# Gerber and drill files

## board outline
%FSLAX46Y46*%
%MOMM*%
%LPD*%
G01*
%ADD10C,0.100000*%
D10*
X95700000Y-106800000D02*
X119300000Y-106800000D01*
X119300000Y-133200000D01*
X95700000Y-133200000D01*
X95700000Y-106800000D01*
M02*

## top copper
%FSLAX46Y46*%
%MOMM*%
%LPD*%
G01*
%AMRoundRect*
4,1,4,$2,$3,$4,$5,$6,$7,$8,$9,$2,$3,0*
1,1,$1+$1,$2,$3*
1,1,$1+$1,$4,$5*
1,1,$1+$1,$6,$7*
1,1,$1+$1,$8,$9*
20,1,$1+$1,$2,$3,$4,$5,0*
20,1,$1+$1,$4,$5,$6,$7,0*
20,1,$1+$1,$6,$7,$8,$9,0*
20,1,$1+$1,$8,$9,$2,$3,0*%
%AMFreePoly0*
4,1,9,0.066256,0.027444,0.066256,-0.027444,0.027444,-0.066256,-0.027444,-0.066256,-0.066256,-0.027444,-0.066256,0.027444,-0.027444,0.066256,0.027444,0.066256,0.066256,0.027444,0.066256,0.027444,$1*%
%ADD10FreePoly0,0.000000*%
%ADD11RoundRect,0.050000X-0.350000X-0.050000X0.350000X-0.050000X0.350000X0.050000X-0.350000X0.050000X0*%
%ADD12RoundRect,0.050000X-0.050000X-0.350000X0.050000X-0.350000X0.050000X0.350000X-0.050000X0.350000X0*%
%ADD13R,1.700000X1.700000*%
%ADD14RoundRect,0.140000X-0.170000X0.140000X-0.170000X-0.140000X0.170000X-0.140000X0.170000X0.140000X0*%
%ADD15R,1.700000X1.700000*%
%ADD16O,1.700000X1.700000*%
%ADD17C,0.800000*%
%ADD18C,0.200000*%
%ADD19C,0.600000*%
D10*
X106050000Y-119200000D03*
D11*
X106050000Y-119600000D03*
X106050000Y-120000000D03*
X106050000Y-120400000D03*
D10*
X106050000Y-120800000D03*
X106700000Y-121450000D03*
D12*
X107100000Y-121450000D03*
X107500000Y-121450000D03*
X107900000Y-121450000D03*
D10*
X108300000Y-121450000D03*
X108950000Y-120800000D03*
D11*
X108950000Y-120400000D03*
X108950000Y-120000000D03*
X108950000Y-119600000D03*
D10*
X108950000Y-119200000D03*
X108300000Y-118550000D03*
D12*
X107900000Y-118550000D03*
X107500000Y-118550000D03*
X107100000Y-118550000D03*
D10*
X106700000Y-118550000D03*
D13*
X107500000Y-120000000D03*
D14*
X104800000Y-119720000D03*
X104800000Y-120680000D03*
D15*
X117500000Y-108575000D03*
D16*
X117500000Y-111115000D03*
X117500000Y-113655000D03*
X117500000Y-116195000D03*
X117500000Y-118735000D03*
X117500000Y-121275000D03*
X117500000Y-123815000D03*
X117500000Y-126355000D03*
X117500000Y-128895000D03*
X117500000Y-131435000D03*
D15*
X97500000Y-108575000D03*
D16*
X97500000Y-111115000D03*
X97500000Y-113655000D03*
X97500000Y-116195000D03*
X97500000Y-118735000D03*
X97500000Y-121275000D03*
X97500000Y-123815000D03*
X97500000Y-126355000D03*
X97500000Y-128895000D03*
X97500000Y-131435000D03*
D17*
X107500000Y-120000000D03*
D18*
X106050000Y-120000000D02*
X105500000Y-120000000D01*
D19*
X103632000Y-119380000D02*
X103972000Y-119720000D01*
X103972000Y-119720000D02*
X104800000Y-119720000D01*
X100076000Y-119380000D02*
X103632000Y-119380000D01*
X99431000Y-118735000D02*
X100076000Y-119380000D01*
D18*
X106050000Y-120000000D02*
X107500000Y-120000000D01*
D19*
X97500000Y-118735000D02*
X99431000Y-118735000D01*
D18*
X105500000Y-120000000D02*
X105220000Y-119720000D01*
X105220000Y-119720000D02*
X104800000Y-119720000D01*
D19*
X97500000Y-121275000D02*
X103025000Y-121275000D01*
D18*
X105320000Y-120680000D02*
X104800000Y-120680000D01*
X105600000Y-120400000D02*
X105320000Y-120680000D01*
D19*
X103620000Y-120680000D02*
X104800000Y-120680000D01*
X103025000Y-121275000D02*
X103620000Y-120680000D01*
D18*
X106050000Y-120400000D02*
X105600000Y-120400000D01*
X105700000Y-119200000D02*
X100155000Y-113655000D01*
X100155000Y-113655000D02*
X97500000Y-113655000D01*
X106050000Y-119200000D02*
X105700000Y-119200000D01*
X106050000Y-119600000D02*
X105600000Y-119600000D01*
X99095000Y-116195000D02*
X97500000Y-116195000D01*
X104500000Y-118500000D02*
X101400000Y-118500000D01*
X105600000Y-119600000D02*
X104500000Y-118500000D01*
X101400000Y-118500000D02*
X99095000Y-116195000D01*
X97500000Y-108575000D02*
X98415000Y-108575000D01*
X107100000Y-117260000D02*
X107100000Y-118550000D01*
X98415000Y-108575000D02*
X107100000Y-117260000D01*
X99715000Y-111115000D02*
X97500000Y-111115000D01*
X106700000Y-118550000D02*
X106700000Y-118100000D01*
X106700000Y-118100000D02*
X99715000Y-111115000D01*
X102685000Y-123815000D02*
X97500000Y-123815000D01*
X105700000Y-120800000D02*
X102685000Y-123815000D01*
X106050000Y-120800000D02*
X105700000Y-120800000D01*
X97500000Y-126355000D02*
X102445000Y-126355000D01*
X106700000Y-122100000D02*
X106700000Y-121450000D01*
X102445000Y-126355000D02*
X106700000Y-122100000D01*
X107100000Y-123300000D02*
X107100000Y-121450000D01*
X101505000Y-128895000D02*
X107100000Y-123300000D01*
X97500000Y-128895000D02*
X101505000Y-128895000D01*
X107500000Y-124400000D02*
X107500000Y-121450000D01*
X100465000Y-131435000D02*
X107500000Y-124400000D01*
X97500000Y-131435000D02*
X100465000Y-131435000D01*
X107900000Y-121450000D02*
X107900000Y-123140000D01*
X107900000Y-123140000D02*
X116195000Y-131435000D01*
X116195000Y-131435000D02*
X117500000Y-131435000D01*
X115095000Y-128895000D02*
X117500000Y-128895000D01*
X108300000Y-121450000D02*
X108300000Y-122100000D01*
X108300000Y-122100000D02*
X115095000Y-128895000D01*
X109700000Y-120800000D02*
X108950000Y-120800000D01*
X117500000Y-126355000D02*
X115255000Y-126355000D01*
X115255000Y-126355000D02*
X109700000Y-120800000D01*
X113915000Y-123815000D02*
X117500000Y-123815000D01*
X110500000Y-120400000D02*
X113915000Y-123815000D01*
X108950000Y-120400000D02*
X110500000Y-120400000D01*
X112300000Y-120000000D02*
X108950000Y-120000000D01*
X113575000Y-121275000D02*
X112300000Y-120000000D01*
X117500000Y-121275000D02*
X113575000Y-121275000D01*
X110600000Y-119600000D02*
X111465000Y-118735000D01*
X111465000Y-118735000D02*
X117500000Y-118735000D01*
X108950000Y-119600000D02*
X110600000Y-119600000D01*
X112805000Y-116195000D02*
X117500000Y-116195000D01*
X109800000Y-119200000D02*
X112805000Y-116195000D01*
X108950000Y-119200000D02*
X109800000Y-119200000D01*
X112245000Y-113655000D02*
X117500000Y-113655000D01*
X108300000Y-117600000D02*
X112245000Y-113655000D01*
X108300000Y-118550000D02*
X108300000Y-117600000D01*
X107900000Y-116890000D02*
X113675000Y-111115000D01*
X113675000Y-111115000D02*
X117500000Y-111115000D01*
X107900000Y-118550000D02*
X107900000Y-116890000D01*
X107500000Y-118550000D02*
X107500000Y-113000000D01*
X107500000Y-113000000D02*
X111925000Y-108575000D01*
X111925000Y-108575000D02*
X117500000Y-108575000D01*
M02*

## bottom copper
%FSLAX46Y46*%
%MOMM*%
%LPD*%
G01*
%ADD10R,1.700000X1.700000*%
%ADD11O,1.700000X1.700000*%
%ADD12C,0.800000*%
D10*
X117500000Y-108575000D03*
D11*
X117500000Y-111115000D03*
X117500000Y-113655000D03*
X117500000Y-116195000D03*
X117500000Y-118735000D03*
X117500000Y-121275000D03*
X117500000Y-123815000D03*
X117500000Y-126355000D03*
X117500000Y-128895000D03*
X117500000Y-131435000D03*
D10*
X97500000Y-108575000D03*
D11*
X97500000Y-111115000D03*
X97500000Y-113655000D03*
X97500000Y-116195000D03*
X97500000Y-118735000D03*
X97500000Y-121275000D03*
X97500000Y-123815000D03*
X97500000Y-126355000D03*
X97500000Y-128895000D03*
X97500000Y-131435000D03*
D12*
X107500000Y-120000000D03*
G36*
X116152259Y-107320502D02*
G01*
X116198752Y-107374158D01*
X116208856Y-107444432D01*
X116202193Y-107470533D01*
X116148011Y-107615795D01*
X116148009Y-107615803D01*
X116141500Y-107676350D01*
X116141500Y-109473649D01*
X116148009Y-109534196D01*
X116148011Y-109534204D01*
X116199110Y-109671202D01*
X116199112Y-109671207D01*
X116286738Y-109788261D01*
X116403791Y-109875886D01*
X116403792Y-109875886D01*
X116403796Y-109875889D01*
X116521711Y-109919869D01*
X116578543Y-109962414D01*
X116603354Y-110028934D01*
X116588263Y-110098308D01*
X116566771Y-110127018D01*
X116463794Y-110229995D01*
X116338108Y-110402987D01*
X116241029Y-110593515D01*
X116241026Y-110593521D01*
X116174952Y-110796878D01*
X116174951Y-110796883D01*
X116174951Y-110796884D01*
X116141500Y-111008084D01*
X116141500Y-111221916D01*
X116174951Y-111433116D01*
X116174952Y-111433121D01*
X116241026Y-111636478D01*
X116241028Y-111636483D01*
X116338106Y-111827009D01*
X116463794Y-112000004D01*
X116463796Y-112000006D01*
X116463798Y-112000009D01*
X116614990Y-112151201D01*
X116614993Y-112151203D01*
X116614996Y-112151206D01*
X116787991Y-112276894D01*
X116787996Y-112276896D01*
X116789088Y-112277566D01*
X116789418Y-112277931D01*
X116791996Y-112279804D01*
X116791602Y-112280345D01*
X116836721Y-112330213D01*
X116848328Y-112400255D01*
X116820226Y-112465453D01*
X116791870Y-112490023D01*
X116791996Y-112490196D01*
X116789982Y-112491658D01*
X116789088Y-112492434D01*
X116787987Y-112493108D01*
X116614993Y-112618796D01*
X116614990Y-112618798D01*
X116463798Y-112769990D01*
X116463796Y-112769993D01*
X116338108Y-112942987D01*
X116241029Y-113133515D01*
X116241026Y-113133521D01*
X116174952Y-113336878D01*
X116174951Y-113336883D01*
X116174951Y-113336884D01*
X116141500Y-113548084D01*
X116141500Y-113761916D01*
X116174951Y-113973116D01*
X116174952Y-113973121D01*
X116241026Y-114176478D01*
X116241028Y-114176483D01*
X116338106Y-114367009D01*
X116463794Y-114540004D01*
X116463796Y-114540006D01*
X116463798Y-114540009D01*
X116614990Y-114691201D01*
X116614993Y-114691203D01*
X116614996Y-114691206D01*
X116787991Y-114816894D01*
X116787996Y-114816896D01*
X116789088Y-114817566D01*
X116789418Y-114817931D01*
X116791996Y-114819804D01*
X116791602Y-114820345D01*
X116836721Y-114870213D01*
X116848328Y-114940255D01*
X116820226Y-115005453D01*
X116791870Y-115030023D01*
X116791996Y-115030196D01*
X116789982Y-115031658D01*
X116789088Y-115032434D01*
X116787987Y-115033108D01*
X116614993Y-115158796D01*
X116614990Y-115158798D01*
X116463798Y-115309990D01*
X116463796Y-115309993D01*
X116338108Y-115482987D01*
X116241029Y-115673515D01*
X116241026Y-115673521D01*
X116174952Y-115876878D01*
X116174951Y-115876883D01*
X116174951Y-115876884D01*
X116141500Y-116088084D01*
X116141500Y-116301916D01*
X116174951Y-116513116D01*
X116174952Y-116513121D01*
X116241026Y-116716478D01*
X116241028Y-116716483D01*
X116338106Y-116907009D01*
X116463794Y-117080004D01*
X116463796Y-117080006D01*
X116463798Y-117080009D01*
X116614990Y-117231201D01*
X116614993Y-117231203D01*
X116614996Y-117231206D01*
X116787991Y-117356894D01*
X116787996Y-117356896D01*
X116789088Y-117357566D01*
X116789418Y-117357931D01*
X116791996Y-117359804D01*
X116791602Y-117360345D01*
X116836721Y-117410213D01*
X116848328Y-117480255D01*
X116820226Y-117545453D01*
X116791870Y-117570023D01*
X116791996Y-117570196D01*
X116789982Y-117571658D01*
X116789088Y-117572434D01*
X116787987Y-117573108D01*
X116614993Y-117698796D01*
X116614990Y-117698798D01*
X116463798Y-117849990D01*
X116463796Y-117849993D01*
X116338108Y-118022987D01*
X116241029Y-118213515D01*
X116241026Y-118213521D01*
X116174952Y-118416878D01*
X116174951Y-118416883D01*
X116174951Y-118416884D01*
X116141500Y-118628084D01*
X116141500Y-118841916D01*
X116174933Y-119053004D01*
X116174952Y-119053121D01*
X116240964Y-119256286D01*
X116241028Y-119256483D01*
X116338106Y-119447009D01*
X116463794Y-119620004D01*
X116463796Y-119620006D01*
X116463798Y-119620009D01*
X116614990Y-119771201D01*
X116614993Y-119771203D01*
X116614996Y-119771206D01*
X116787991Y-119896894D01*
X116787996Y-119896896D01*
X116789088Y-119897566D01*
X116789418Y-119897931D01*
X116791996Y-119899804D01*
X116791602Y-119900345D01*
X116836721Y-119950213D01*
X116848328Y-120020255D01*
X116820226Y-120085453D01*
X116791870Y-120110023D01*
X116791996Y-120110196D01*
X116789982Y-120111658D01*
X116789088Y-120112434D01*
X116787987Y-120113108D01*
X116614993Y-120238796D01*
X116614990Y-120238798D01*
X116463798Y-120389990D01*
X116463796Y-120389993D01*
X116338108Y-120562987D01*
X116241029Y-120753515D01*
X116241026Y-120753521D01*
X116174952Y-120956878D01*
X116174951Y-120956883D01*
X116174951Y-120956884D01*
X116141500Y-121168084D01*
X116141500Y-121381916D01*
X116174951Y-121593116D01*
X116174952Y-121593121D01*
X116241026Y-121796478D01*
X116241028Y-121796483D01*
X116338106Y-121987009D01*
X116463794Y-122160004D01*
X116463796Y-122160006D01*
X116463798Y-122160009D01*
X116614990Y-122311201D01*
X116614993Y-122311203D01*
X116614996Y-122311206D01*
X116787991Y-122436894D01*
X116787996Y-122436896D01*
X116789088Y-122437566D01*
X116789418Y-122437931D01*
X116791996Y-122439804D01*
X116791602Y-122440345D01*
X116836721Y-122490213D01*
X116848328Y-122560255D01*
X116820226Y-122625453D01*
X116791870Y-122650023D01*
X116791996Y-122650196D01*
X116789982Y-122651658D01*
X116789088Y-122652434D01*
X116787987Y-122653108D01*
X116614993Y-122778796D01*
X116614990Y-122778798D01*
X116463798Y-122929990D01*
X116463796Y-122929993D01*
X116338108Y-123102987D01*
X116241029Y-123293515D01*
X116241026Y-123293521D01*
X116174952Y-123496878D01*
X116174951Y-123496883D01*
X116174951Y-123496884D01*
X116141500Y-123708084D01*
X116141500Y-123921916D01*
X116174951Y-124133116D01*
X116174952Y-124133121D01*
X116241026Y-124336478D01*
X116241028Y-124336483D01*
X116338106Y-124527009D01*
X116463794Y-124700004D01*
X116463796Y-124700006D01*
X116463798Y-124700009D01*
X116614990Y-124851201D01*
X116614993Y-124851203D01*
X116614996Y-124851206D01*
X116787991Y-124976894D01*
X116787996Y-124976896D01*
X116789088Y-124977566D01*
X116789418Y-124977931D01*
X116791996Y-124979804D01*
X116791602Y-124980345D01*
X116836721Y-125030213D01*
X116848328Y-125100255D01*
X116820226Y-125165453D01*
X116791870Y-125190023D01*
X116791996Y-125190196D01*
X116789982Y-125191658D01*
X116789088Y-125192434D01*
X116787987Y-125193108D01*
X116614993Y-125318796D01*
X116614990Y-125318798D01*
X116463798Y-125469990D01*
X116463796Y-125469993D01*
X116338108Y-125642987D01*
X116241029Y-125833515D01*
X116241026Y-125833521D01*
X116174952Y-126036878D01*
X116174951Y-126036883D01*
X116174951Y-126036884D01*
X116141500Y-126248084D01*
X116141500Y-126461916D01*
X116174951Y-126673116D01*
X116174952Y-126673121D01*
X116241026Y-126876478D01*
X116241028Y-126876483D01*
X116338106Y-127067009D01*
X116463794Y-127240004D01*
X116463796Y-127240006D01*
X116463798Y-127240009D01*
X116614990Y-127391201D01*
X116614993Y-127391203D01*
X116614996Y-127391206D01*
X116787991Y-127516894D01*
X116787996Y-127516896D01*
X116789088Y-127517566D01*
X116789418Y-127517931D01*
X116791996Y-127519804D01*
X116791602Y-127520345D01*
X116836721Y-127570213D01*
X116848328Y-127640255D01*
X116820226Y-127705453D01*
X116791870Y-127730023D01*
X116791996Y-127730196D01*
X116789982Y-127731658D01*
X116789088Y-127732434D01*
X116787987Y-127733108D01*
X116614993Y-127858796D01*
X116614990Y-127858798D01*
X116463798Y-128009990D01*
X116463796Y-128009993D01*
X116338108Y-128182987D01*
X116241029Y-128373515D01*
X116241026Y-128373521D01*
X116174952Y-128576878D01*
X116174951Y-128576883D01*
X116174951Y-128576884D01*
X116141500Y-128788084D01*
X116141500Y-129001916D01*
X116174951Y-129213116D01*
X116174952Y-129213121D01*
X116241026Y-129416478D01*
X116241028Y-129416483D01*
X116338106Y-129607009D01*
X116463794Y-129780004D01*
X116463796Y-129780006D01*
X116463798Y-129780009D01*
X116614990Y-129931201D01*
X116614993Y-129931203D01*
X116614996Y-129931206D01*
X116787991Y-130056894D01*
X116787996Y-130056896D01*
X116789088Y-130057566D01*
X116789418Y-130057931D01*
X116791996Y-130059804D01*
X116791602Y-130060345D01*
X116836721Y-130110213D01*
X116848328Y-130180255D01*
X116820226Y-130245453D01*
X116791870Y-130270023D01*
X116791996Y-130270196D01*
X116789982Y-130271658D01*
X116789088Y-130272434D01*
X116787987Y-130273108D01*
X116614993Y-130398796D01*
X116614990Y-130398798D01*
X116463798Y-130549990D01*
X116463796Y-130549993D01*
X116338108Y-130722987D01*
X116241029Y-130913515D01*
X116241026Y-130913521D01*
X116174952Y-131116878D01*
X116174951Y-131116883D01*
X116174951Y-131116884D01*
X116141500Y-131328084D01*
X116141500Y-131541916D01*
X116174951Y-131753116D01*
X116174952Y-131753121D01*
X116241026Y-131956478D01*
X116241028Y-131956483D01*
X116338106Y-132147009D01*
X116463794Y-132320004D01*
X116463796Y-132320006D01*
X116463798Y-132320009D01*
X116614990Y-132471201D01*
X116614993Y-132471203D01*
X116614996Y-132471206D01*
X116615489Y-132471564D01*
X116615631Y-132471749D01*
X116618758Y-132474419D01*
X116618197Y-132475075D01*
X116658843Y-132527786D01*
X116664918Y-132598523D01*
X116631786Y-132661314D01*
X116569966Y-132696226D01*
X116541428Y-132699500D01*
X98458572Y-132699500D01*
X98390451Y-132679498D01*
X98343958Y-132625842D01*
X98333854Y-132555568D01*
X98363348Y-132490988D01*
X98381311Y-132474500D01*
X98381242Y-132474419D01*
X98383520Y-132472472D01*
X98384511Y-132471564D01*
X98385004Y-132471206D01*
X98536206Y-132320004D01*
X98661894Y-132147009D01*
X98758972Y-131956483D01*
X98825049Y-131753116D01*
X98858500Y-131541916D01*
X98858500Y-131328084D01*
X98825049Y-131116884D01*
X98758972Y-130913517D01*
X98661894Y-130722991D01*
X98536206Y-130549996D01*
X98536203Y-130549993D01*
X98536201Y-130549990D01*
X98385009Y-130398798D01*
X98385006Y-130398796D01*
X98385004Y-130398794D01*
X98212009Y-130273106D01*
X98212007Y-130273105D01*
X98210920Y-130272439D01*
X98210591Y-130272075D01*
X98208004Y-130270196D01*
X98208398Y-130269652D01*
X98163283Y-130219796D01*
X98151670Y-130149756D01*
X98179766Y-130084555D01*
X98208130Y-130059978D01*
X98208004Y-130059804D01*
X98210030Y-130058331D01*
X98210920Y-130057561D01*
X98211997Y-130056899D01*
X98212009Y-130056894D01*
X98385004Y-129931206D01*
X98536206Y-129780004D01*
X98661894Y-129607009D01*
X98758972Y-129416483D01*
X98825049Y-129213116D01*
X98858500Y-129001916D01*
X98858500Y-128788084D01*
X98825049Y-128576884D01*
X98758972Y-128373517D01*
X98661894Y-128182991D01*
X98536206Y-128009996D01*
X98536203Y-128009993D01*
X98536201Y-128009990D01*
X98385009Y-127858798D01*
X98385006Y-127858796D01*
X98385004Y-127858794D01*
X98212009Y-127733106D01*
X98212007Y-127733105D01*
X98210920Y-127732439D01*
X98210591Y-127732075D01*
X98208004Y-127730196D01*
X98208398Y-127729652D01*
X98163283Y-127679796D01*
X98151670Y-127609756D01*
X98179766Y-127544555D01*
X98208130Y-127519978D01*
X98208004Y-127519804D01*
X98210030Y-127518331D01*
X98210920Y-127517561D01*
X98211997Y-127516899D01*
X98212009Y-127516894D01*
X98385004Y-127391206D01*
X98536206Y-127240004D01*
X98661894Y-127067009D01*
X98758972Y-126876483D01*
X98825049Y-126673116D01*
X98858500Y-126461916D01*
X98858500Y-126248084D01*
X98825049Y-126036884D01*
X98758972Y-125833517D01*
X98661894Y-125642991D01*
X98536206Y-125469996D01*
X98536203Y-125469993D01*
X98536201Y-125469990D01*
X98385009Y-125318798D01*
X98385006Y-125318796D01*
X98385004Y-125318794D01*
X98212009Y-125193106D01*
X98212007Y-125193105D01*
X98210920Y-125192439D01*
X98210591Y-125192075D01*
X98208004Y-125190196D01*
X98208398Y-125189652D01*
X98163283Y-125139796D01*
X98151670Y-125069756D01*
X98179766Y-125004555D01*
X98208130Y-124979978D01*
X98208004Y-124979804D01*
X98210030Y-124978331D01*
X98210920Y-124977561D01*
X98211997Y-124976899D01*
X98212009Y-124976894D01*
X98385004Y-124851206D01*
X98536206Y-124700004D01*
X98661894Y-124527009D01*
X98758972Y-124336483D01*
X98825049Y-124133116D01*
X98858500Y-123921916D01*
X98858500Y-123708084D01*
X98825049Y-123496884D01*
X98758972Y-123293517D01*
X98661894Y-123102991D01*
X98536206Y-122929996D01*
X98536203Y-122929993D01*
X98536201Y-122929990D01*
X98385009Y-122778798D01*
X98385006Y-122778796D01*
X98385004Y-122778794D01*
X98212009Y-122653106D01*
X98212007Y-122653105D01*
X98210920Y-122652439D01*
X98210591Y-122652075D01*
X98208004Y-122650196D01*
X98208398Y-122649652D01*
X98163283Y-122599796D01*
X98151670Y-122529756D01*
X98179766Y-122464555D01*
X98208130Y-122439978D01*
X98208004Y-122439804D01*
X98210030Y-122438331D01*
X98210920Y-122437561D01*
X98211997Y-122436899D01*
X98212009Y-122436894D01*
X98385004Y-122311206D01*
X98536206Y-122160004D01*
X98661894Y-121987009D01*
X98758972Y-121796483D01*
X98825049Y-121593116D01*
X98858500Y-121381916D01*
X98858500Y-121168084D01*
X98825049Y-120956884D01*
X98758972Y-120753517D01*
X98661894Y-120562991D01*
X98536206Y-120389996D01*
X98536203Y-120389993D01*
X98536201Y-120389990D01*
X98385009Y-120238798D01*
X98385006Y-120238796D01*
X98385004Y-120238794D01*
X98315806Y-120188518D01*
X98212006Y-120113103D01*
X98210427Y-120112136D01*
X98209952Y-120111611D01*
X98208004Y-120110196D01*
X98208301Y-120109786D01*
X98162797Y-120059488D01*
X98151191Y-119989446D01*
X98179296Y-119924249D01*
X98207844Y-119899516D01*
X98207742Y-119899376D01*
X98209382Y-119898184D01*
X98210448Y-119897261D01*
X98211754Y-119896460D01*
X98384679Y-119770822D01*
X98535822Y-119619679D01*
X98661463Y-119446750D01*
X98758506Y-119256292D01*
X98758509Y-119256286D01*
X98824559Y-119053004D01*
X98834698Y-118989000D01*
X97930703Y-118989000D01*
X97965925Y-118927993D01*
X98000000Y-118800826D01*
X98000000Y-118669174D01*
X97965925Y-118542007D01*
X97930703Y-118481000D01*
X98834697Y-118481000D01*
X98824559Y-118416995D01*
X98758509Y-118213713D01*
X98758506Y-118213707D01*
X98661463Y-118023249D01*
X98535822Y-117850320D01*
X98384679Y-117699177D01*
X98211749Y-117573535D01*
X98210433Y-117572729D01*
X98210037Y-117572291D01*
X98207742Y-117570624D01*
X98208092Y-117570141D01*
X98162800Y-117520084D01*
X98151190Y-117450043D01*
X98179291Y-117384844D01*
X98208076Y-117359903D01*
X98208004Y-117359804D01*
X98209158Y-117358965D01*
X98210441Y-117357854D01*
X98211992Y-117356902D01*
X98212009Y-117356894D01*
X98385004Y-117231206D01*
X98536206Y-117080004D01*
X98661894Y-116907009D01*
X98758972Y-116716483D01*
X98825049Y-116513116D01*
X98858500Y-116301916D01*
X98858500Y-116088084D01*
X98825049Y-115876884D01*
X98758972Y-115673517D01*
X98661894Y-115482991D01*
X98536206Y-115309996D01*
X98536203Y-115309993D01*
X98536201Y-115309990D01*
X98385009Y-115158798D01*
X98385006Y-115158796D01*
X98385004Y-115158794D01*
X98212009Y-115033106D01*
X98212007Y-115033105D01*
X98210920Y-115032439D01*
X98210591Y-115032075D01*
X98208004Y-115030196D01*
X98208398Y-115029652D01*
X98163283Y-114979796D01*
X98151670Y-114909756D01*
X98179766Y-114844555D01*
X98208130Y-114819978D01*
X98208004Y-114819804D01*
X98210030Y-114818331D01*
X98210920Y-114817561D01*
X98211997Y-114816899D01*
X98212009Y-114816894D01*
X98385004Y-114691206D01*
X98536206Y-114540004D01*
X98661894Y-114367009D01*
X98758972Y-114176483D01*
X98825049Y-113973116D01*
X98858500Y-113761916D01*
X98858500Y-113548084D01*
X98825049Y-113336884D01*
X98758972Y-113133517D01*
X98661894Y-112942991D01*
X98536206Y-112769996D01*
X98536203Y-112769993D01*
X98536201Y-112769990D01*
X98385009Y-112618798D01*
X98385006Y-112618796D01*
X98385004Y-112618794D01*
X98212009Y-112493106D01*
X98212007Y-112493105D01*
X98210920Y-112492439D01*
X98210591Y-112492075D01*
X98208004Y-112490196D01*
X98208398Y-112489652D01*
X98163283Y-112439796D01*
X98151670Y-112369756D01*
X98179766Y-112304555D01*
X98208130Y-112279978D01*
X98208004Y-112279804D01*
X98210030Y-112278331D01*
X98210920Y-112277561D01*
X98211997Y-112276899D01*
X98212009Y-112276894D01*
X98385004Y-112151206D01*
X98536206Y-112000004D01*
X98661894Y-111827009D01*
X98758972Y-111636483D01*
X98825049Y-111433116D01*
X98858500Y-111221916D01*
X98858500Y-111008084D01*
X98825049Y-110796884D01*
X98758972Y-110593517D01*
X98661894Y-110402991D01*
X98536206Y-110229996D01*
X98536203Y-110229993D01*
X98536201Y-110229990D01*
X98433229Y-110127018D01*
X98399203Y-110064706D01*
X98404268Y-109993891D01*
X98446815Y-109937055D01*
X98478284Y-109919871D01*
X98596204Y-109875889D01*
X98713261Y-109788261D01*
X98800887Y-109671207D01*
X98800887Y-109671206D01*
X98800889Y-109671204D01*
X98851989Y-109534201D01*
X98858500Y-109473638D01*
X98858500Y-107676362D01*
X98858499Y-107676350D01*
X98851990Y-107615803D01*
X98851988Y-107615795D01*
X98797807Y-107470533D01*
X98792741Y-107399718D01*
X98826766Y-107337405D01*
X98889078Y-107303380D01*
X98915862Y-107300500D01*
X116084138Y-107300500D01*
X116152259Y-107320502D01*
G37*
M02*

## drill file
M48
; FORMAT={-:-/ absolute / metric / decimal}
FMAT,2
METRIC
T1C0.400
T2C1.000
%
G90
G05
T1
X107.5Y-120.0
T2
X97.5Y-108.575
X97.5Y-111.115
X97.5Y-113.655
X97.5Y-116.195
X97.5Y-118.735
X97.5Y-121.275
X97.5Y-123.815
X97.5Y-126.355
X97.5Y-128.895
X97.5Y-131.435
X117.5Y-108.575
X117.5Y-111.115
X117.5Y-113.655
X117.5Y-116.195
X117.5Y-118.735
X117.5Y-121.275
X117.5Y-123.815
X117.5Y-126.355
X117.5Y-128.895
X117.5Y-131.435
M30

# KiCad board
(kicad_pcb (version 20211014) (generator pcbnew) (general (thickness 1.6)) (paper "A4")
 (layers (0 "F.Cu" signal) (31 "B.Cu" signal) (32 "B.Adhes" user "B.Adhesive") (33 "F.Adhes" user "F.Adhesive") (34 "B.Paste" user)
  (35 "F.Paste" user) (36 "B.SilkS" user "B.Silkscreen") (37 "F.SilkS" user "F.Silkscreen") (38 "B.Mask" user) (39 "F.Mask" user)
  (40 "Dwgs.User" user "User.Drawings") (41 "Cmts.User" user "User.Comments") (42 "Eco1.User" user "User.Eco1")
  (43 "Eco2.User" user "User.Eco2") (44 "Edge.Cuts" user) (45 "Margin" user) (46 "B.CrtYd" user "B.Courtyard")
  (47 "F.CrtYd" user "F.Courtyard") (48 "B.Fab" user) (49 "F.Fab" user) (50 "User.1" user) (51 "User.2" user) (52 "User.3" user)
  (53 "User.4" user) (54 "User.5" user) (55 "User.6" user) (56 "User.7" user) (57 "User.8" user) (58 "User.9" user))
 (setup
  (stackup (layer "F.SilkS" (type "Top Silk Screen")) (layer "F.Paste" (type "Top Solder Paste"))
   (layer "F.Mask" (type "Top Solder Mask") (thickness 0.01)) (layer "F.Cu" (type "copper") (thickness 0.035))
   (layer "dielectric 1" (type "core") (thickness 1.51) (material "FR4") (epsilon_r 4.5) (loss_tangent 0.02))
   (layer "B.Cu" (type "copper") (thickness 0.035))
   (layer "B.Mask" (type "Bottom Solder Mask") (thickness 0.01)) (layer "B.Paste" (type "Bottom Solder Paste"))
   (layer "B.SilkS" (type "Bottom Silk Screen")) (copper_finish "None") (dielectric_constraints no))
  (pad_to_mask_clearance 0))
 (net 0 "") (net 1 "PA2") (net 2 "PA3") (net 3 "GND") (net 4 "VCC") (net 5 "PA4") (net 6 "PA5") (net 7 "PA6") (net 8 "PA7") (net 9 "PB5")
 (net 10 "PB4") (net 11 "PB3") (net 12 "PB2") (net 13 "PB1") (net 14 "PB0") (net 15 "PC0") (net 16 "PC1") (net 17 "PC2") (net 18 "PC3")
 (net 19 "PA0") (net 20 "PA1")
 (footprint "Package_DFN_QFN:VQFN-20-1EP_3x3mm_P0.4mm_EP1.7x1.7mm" (layer "F.Cu") (at 107.5 120)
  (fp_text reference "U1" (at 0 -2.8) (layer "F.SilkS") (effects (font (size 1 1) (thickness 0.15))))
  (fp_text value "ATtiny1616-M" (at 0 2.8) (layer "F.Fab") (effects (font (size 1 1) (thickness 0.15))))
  (pad "" smd roundrect (at 0.425 -0.425) (size 0.69 0.69) (layers "F.Paste") (roundrect_rratio 0.25))
  (pad "" smd roundrect (at -0.425 -0.425) (size 0.69 0.69) (layers "F.Paste") (roundrect_rratio 0.25))
  (pad "" smd roundrect (at 0.425 0.425) (size 0.69 0.69) (layers "F.Paste") (roundrect_rratio 0.25))
  (pad "" smd roundrect (at -0.425 0.425) (size 0.69 0.69) (layers "F.Paste") (roundrect_rratio 0.25))
  (pad "1" smd custom (at -1.45 -0.8) (size 0.143431 0.143431) (layers "F.Cu" "F.Paste" "F.Mask") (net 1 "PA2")
   (options (clearance outline) (anchor circle)) (primitives))
  (pad "2" smd roundrect (at -1.45 -0.4) (size 0.8 0.2) (layers "F.Cu" "F.Paste" "F.Mask") (roundrect_rratio 0.25) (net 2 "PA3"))
  (pad "3" smd roundrect (at -1.45 0) (size 0.8 0.2) (layers "F.Cu" "F.Paste" "F.Mask") (roundrect_rratio 0.25) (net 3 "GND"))
  (pad "4" smd roundrect (at -1.45 0.4) (size 0.8 0.2) (layers "F.Cu" "F.Paste" "F.Mask") (roundrect_rratio 0.25) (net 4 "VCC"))
  (pad "5" smd custom (at -1.45 0.8) (size 0.143431 0.143431) (layers "F.Cu" "F.Paste" "F.Mask") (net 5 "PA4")
   (options (clearance outline) (anchor circle)) (primitives))
  (pad "6" smd custom (at -0.8 1.45) (size 0.143431 0.143431) (layers "F.Cu" "F.Paste" "F.Mask") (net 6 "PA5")
   (options (clearance outline) (anchor circle)) (primitives))
  (pad "7" smd roundrect (at -0.4 1.45) (size 0.2 0.8) (layers "F.Cu" "F.Paste" "F.Mask") (roundrect_rratio 0.25) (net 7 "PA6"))
  (pad "8" smd roundrect (at 0 1.45) (size 0.2 0.8) (layers "F.Cu" "F.Paste" "F.Mask") (roundrect_rratio 0.25) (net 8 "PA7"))
  (pad "9" smd roundrect (at 0.4 1.45) (size 0.2 0.8) (layers "F.Cu" "F.Paste" "F.Mask") (roundrect_rratio 0.25) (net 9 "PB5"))
  (pad "10" smd custom (at 0.8 1.45) (size 0.143431 0.143431) (layers "F.Cu" "F.Paste" "F.Mask") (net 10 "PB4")
   (options (clearance outline) (anchor circle)) (primitives))
  (pad "11" smd custom (at 1.45 0.8) (size 0.143431 0.143431) (layers "F.Cu" "F.Paste" "F.Mask") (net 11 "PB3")
   (options (clearance outline) (anchor circle)) (primitives))
  (pad "12" smd roundrect (at 1.45 0.4) (size 0.8 0.2) (layers "F.Cu" "F.Paste" "F.Mask") (roundrect_rratio 0.25) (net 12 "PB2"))
  (pad "13" smd roundrect (at 1.45 0) (size 0.8 0.2) (layers "F.Cu" "F.Paste" "F.Mask") (roundrect_rratio 0.25) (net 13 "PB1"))
  (pad "14" smd roundrect (at 1.45 -0.4) (size 0.8 0.2) (layers "F.Cu" "F.Paste" "F.Mask") (roundrect_rratio 0.25) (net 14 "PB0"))
  (pad "15" smd custom (at 1.45 -0.8) (size 0.143431 0.143431) (layers "F.Cu" "F.Paste" "F.Mask") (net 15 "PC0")
   (options (clearance outline) (anchor circle)) (primitives))
  (pad "16" smd custom (at 0.8 -1.45) (size 0.143431 0.143431) (layers "F.Cu" "F.Paste" "F.Mask") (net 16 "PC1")
   (options (clearance outline) (anchor circle)) (primitives))
  (pad "17" smd roundrect (at 0.4 -1.45) (size 0.2 0.8) (layers "F.Cu" "F.Paste" "F.Mask") (roundrect_rratio 0.25) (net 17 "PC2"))
  (pad "18" smd roundrect (at 0 -1.45) (size 0.2 0.8) (layers "F.Cu" "F.Paste" "F.Mask") (roundrect_rratio 0.25) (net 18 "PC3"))
  (pad "19" smd roundrect (at -0.4 -1.45) (size 0.2 0.8) (layers "F.Cu" "F.Paste" "F.Mask") (roundrect_rratio 0.25) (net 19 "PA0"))
  (pad "20" smd custom (at -0.8 -1.45) (size 0.143431 0.143431) (layers "F.Cu" "F.Paste" "F.Mask") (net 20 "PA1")
   (options (clearance outline) (anchor circle)) (primitives))
  (pad "21" smd rect (at 0 0) (size 1.7 1.7) (layers "F.Cu" "F.Mask") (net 3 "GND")))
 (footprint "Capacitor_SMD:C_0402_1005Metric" (layer "F.Cu") (at 104.8 120.2 -90)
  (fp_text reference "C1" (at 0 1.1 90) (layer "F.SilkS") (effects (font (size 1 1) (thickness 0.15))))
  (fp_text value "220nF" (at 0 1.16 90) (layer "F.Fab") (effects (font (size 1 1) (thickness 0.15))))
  (pad "1" smd roundrect (at -0.48 0 270) (size 0.56 0.62) (layers "F.Cu" "F.Paste" "F.Mask") (roundrect_rratio 0.25) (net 3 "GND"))
  (pad "2" smd roundrect (at 0.48 0 270) (size 0.56 0.62) (layers "F.Cu" "F.Paste" "F.Mask") (roundrect_rratio 0.25) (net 4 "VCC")))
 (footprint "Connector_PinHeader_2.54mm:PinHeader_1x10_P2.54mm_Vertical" (layer "B.Cu") (at 117.5 108.575 180)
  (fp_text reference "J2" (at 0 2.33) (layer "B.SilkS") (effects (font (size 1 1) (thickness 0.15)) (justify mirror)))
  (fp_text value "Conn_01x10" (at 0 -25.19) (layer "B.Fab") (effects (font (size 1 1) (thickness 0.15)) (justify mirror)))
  (pad "1" thru_hole rect (at 0 0 180) (size 1.7 1.7) (drill 1) (layers *.Cu *.Mask) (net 18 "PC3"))
  (pad "2" thru_hole oval (at 0 -2.54 180) (size 1.7 1.7) (drill 1) (layers *.Cu *.Mask) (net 17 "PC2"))
  (pad "3" thru_hole oval (at 0 -5.08 180) (size 1.7 1.7) (drill 1) (layers *.Cu *.Mask) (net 16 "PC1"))
  (pad "4" thru_hole oval (at 0 -7.62 180) (size 1.7 1.7) (drill 1) (layers *.Cu *.Mask) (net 15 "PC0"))
  (pad "5" thru_hole oval (at 0 -10.16 180) (size 1.7 1.7) (drill 1) (layers *.Cu *.Mask) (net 14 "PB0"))
  (pad "6" thru_hole oval (at 0 -12.7 180) (size 1.7 1.7) (drill 1) (layers *.Cu *.Mask) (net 13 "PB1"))
  (pad "7" thru_hole oval (at 0 -15.24 180) (size 1.7 1.7) (drill 1) (layers *.Cu *.Mask) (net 12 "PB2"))
  (pad "8" thru_hole oval (at 0 -17.78 180) (size 1.7 1.7) (drill 1) (layers *.Cu *.Mask) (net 11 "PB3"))
  (pad "9" thru_hole oval (at 0 -20.32 180) (size 1.7 1.7) (drill 1) (layers *.Cu *.Mask) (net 10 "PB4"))
  (pad "10" thru_hole oval (at 0 -22.86 180) (size 1.7 1.7) (drill 1) (layers *.Cu *.Mask) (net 9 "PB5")))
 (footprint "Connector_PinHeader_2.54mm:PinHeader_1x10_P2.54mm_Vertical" (layer "B.Cu") (at 97.5 108.575 180)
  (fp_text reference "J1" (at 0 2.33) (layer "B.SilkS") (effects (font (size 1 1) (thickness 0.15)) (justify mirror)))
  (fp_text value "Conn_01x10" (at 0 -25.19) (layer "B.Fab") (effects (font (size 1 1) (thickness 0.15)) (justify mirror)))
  (pad "1" thru_hole rect (at 0 0 180) (size 1.7 1.7) (drill 1) (layers *.Cu *.Mask) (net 19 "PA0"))
  (pad "2" thru_hole oval (at 0 -2.54 180) (size 1.7 1.7) (drill 1) (layers *.Cu *.Mask) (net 20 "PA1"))
  (pad "3" thru_hole oval (at 0 -5.08 180) (size 1.7 1.7) (drill 1) (layers *.Cu *.Mask) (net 1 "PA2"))
  (pad "4" thru_hole oval (at 0 -7.62 180) (size 1.7 1.7) (drill 1) (layers *.Cu *.Mask) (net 2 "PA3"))
  (pad "5" thru_hole oval (at 0 -10.16 180) (size 1.7 1.7) (drill 1) (layers *.Cu *.Mask) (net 3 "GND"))
  (pad "6" thru_hole oval (at 0 -12.7 180) (size 1.7 1.7) (drill 1) (layers *.Cu *.Mask) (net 4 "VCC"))
  (pad "7" thru_hole oval (at 0 -15.24 180) (size 1.7 1.7) (drill 1) (layers *.Cu *.Mask) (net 5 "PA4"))
  (pad "8" thru_hole oval (at 0 -17.78 180) (size 1.7 1.7) (drill 1) (layers *.Cu *.Mask) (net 6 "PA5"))
  (pad "9" thru_hole oval (at 0 -20.32 180) (size 1.7 1.7) (drill 1) (layers *.Cu *.Mask) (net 7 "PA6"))
  (pad "10" thru_hole oval (at 0 -22.86 180) (size 1.7 1.7) (drill 1) (layers *.Cu *.Mask) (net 8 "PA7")))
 (gr_rect (start 95.7 106.8) (end 119.3 133.2) (layer "Edge.Cuts") (width 0.1) (fill none))
 (segment (start 106.05 120) (end 105.5 120) (width 0.2) (layer "F.Cu") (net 3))
 (segment (start 103.632 119.38) (end 103.972 119.72) (width 0.6) (layer "F.Cu") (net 3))
 (segment (start 103.972 119.72) (end 104.8 119.72) (width 0.6) (layer "F.Cu") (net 3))
 (segment (start 100.076 119.38) (end 103.632 119.38) (width 0.6) (layer "F.Cu") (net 3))
 (segment (start 99.431 118.735) (end 100.076 119.38) (width 0.6) (layer "F.Cu") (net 3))
 (segment (start 106.05 120) (end 107.5 120) (width 0.2) (layer "F.Cu") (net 3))
 (segment (start 97.5 118.735) (end 99.431 118.735) (width 0.6) (layer "F.Cu") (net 3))
 (segment (start 105.5 120) (end 105.22 119.72) (width 0.2) (layer "F.Cu") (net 3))
 (segment (start 105.22 119.72) (end 104.8 119.72) (width 0.2) (layer "F.Cu") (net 3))
 (via (at 107.5 120) (size 0.8) (drill 0.4) (layers "F.Cu" "B.Cu") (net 3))
 (segment (start 97.5 121.275) (end 103.025 121.275) (width 0.6) (layer "F.Cu") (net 4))
 (segment (start 105.32 120.68) (end 104.8 120.68) (width 0.2) (layer "F.Cu") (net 4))
 (segment (start 105.6 120.4) (end 105.32 120.68) (width 0.2) (layer "F.Cu") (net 4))
 (segment (start 103.62 120.68) (end 104.8 120.68) (width 0.6) (layer "F.Cu") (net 4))
 (segment (start 103.025 121.275) (end 103.62 120.68) (width 0.6) (layer "F.Cu") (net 4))
 (segment (start 106.05 120.4) (end 105.6 120.4) (width 0.2) (layer "F.Cu") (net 4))
 (segment (start 105.7 119.2) (end 100.155 113.655) (width 0.2) (layer "F.Cu") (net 1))
 (segment (start 100.155 113.655) (end 97.5 113.655) (width 0.2) (layer "F.Cu") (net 1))
 (segment (start 106.05 119.2) (end 105.7 119.2) (width 0.2) (layer "F.Cu") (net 1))
 (segment (start 106.05 119.6) (end 105.6 119.6) (width 0.2) (layer "F.Cu") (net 2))
 (segment (start 99.095 116.195) (end 97.5 116.195) (width 0.2) (layer "F.Cu") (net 2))
 (segment (start 104.5 118.5) (end 101.4 118.5) (width 0.2) (layer "F.Cu") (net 2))
 (segment (start 105.6 119.6) (end 104.5 118.5) (width 0.2) (layer "F.Cu") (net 2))
 (segment (start 101.4 118.5) (end 99.095 116.195) (width 0.2) (layer "F.Cu") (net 2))
 (segment (start 97.5 108.575) (end 98.415 108.575) (width 0.2) (layer "F.Cu") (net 19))
 (segment (start 107.1 117.26) (end 107.1 118.55) (width 0.2) (layer "F.Cu") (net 19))
 (segment (start 98.415 108.575) (end 107.1 117.26) (width 0.2) (layer "F.Cu") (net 19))
 (segment (start 99.715 111.115) (end 97.5 111.115) (width 0.2) (layer "F.Cu") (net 20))
 (segment (start 106.7 118.55) (end 106.7 118.1) (width 0.2) (layer "F.Cu") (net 20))
 (segment (start 106.7 118.1) (end 99.715 111.115) (width 0.2) (layer "F.Cu") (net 20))
 (segment (start 102.685 123.815) (end 97.5 123.815) (width 0.2) (layer "F.Cu") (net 5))
 (segment (start 105.7 120.8) (end 102.685 123.815) (width 0.2) (layer "F.Cu") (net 5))
 (segment (start 106.05 120.8) (end 105.7 120.8) (width 0.2) (layer "F.Cu") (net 5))
 (segment (start 97.5 126.355) (end 102.445 126.355) (width 0.2) (layer "F.Cu") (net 6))
 (segment (start 106.7 122.1) (end 106.7 121.45) (width 0.2) (layer "F.Cu") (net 6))
 (segment (start 102.445 126.355) (end 106.7 122.1) (width 0.2) (layer "F.Cu") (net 6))
 (segment (start 107.1 123.3) (end 107.1 121.45) (width 0.2) (layer "F.Cu") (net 7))
 (segment (start 101.505 128.895) (end 107.1 123.3) (width 0.2) (layer "F.Cu") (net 7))
 (segment (start 97.5 128.895) (end 101.505 128.895) (width 0.2) (layer "F.Cu") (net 7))
 (segment (start 107.5 124.4) (end 107.5 121.45) (width 0.2) (layer "F.Cu") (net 8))
 (segment (start 100.465 131.435) (end 107.5 124.4) (width 0.2) (layer "F.Cu") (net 8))
 (segment (start 97.5 131.435) (end 100.465 131.435) (width 0.2) (layer "F.Cu") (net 8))
 (segment (start 107.9 121.45) (end 107.9 123.14) (width 0.2) (layer "F.Cu") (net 9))
 (segment (start 107.9 123.14) (end 116.195 131.435) (width 0.2) (layer "F.Cu") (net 9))
 (segment (start 116.195 131.435) (end 117.5 131.435) (width 0.2) (layer "F.Cu") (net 9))
 (segment (start 115.095 128.895) (end 117.5 128.895) (width 0.2) (layer "F.Cu") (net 10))
 (segment (start 108.3 121.45) (end 108.3 122.1) (width 0.2) (layer "F.Cu") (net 10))
 (segment (start 108.3 122.1) (end 115.095 128.895) (width 0.2) (layer "F.Cu") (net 10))
 (segment (start 109.7 120.8) (end 108.95 120.8) (width 0.2) (layer "F.Cu") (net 11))
 (segment (start 117.5 126.355) (end 115.255 126.355) (width 0.2) (layer "F.Cu") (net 11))
 (segment (start 115.255 126.355) (end 109.7 120.8) (width 0.2) (layer "F.Cu") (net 11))
 (segment (start 113.915 123.815) (end 117.5 123.815) (width 0.2) (layer "F.Cu") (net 12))
 (segment (start 110.5 120.4) (end 113.915 123.815) (width 0.2) (layer "F.Cu") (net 12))
 (segment (start 108.95 120.4) (end 110.5 120.4) (width 0.2) (layer "F.Cu") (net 12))
 (segment (start 112.3 120) (end 108.95 120) (width 0.2) (layer "F.Cu") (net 13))
 (segment (start 113.575 121.275) (end 112.3 120) (width 0.2) (layer "F.Cu") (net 13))
 (segment (start 117.5 121.275) (end 113.575 121.275) (width 0.2) (layer "F.Cu") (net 13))
 (segment (start 110.6 119.6) (end 111.465 118.735) (width 0.2) (layer "F.Cu") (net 14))
 (segment (start 111.465 118.735) (end 117.5 118.735) (width 0.2) (layer "F.Cu") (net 14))
 (segment (start 108.95 119.6) (end 110.6 119.6) (width 0.2) (layer "F.Cu") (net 14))
 (segment (start 112.805 116.195) (end 117.5 116.195) (width 0.2) (layer "F.Cu") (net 15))
 (segment (start 109.8 119.2) (end 112.805 116.195) (width 0.2) (layer "F.Cu") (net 15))
 (segment (start 108.95 119.2) (end 109.8 119.2) (width 0.2) (layer "F.Cu") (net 15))
 (segment (start 112.245 113.655) (end 117.5 113.655) (width 0.2) (layer "F.Cu") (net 16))
 (segment (start 108.3 117.6) (end 112.245 113.655) (width 0.2) (layer "F.Cu") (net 16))
 (segment (start 108.3 118.55) (end 108.3 117.6) (width 0.2) (layer "F.Cu") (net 16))
 (segment (start 107.9 116.89) (end 113.675 111.115) (width 0.2) (layer "F.Cu") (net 17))
 (segment (start 113.675 111.115) (end 117.5 111.115) (width 0.2) (layer "F.Cu") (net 17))
 (segment (start 107.9 118.55) (end 107.9 116.89) (width 0.2) (layer "F.Cu") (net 17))
 (segment (start 107.5 118.55) (end 107.5 113) (width 0.2) (layer "F.Cu") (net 18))
 (segment (start 107.5 113) (end 111.925 108.575) (width 0.2) (layer "F.Cu") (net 18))
 (segment (start 111.925 108.575) (end 117.5 108.575) (width 0.2) (layer "F.Cu") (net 18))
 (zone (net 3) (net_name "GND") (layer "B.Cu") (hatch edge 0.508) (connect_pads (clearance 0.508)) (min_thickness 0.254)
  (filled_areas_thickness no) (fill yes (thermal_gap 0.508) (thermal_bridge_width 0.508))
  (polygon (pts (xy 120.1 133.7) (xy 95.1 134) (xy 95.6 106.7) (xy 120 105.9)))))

